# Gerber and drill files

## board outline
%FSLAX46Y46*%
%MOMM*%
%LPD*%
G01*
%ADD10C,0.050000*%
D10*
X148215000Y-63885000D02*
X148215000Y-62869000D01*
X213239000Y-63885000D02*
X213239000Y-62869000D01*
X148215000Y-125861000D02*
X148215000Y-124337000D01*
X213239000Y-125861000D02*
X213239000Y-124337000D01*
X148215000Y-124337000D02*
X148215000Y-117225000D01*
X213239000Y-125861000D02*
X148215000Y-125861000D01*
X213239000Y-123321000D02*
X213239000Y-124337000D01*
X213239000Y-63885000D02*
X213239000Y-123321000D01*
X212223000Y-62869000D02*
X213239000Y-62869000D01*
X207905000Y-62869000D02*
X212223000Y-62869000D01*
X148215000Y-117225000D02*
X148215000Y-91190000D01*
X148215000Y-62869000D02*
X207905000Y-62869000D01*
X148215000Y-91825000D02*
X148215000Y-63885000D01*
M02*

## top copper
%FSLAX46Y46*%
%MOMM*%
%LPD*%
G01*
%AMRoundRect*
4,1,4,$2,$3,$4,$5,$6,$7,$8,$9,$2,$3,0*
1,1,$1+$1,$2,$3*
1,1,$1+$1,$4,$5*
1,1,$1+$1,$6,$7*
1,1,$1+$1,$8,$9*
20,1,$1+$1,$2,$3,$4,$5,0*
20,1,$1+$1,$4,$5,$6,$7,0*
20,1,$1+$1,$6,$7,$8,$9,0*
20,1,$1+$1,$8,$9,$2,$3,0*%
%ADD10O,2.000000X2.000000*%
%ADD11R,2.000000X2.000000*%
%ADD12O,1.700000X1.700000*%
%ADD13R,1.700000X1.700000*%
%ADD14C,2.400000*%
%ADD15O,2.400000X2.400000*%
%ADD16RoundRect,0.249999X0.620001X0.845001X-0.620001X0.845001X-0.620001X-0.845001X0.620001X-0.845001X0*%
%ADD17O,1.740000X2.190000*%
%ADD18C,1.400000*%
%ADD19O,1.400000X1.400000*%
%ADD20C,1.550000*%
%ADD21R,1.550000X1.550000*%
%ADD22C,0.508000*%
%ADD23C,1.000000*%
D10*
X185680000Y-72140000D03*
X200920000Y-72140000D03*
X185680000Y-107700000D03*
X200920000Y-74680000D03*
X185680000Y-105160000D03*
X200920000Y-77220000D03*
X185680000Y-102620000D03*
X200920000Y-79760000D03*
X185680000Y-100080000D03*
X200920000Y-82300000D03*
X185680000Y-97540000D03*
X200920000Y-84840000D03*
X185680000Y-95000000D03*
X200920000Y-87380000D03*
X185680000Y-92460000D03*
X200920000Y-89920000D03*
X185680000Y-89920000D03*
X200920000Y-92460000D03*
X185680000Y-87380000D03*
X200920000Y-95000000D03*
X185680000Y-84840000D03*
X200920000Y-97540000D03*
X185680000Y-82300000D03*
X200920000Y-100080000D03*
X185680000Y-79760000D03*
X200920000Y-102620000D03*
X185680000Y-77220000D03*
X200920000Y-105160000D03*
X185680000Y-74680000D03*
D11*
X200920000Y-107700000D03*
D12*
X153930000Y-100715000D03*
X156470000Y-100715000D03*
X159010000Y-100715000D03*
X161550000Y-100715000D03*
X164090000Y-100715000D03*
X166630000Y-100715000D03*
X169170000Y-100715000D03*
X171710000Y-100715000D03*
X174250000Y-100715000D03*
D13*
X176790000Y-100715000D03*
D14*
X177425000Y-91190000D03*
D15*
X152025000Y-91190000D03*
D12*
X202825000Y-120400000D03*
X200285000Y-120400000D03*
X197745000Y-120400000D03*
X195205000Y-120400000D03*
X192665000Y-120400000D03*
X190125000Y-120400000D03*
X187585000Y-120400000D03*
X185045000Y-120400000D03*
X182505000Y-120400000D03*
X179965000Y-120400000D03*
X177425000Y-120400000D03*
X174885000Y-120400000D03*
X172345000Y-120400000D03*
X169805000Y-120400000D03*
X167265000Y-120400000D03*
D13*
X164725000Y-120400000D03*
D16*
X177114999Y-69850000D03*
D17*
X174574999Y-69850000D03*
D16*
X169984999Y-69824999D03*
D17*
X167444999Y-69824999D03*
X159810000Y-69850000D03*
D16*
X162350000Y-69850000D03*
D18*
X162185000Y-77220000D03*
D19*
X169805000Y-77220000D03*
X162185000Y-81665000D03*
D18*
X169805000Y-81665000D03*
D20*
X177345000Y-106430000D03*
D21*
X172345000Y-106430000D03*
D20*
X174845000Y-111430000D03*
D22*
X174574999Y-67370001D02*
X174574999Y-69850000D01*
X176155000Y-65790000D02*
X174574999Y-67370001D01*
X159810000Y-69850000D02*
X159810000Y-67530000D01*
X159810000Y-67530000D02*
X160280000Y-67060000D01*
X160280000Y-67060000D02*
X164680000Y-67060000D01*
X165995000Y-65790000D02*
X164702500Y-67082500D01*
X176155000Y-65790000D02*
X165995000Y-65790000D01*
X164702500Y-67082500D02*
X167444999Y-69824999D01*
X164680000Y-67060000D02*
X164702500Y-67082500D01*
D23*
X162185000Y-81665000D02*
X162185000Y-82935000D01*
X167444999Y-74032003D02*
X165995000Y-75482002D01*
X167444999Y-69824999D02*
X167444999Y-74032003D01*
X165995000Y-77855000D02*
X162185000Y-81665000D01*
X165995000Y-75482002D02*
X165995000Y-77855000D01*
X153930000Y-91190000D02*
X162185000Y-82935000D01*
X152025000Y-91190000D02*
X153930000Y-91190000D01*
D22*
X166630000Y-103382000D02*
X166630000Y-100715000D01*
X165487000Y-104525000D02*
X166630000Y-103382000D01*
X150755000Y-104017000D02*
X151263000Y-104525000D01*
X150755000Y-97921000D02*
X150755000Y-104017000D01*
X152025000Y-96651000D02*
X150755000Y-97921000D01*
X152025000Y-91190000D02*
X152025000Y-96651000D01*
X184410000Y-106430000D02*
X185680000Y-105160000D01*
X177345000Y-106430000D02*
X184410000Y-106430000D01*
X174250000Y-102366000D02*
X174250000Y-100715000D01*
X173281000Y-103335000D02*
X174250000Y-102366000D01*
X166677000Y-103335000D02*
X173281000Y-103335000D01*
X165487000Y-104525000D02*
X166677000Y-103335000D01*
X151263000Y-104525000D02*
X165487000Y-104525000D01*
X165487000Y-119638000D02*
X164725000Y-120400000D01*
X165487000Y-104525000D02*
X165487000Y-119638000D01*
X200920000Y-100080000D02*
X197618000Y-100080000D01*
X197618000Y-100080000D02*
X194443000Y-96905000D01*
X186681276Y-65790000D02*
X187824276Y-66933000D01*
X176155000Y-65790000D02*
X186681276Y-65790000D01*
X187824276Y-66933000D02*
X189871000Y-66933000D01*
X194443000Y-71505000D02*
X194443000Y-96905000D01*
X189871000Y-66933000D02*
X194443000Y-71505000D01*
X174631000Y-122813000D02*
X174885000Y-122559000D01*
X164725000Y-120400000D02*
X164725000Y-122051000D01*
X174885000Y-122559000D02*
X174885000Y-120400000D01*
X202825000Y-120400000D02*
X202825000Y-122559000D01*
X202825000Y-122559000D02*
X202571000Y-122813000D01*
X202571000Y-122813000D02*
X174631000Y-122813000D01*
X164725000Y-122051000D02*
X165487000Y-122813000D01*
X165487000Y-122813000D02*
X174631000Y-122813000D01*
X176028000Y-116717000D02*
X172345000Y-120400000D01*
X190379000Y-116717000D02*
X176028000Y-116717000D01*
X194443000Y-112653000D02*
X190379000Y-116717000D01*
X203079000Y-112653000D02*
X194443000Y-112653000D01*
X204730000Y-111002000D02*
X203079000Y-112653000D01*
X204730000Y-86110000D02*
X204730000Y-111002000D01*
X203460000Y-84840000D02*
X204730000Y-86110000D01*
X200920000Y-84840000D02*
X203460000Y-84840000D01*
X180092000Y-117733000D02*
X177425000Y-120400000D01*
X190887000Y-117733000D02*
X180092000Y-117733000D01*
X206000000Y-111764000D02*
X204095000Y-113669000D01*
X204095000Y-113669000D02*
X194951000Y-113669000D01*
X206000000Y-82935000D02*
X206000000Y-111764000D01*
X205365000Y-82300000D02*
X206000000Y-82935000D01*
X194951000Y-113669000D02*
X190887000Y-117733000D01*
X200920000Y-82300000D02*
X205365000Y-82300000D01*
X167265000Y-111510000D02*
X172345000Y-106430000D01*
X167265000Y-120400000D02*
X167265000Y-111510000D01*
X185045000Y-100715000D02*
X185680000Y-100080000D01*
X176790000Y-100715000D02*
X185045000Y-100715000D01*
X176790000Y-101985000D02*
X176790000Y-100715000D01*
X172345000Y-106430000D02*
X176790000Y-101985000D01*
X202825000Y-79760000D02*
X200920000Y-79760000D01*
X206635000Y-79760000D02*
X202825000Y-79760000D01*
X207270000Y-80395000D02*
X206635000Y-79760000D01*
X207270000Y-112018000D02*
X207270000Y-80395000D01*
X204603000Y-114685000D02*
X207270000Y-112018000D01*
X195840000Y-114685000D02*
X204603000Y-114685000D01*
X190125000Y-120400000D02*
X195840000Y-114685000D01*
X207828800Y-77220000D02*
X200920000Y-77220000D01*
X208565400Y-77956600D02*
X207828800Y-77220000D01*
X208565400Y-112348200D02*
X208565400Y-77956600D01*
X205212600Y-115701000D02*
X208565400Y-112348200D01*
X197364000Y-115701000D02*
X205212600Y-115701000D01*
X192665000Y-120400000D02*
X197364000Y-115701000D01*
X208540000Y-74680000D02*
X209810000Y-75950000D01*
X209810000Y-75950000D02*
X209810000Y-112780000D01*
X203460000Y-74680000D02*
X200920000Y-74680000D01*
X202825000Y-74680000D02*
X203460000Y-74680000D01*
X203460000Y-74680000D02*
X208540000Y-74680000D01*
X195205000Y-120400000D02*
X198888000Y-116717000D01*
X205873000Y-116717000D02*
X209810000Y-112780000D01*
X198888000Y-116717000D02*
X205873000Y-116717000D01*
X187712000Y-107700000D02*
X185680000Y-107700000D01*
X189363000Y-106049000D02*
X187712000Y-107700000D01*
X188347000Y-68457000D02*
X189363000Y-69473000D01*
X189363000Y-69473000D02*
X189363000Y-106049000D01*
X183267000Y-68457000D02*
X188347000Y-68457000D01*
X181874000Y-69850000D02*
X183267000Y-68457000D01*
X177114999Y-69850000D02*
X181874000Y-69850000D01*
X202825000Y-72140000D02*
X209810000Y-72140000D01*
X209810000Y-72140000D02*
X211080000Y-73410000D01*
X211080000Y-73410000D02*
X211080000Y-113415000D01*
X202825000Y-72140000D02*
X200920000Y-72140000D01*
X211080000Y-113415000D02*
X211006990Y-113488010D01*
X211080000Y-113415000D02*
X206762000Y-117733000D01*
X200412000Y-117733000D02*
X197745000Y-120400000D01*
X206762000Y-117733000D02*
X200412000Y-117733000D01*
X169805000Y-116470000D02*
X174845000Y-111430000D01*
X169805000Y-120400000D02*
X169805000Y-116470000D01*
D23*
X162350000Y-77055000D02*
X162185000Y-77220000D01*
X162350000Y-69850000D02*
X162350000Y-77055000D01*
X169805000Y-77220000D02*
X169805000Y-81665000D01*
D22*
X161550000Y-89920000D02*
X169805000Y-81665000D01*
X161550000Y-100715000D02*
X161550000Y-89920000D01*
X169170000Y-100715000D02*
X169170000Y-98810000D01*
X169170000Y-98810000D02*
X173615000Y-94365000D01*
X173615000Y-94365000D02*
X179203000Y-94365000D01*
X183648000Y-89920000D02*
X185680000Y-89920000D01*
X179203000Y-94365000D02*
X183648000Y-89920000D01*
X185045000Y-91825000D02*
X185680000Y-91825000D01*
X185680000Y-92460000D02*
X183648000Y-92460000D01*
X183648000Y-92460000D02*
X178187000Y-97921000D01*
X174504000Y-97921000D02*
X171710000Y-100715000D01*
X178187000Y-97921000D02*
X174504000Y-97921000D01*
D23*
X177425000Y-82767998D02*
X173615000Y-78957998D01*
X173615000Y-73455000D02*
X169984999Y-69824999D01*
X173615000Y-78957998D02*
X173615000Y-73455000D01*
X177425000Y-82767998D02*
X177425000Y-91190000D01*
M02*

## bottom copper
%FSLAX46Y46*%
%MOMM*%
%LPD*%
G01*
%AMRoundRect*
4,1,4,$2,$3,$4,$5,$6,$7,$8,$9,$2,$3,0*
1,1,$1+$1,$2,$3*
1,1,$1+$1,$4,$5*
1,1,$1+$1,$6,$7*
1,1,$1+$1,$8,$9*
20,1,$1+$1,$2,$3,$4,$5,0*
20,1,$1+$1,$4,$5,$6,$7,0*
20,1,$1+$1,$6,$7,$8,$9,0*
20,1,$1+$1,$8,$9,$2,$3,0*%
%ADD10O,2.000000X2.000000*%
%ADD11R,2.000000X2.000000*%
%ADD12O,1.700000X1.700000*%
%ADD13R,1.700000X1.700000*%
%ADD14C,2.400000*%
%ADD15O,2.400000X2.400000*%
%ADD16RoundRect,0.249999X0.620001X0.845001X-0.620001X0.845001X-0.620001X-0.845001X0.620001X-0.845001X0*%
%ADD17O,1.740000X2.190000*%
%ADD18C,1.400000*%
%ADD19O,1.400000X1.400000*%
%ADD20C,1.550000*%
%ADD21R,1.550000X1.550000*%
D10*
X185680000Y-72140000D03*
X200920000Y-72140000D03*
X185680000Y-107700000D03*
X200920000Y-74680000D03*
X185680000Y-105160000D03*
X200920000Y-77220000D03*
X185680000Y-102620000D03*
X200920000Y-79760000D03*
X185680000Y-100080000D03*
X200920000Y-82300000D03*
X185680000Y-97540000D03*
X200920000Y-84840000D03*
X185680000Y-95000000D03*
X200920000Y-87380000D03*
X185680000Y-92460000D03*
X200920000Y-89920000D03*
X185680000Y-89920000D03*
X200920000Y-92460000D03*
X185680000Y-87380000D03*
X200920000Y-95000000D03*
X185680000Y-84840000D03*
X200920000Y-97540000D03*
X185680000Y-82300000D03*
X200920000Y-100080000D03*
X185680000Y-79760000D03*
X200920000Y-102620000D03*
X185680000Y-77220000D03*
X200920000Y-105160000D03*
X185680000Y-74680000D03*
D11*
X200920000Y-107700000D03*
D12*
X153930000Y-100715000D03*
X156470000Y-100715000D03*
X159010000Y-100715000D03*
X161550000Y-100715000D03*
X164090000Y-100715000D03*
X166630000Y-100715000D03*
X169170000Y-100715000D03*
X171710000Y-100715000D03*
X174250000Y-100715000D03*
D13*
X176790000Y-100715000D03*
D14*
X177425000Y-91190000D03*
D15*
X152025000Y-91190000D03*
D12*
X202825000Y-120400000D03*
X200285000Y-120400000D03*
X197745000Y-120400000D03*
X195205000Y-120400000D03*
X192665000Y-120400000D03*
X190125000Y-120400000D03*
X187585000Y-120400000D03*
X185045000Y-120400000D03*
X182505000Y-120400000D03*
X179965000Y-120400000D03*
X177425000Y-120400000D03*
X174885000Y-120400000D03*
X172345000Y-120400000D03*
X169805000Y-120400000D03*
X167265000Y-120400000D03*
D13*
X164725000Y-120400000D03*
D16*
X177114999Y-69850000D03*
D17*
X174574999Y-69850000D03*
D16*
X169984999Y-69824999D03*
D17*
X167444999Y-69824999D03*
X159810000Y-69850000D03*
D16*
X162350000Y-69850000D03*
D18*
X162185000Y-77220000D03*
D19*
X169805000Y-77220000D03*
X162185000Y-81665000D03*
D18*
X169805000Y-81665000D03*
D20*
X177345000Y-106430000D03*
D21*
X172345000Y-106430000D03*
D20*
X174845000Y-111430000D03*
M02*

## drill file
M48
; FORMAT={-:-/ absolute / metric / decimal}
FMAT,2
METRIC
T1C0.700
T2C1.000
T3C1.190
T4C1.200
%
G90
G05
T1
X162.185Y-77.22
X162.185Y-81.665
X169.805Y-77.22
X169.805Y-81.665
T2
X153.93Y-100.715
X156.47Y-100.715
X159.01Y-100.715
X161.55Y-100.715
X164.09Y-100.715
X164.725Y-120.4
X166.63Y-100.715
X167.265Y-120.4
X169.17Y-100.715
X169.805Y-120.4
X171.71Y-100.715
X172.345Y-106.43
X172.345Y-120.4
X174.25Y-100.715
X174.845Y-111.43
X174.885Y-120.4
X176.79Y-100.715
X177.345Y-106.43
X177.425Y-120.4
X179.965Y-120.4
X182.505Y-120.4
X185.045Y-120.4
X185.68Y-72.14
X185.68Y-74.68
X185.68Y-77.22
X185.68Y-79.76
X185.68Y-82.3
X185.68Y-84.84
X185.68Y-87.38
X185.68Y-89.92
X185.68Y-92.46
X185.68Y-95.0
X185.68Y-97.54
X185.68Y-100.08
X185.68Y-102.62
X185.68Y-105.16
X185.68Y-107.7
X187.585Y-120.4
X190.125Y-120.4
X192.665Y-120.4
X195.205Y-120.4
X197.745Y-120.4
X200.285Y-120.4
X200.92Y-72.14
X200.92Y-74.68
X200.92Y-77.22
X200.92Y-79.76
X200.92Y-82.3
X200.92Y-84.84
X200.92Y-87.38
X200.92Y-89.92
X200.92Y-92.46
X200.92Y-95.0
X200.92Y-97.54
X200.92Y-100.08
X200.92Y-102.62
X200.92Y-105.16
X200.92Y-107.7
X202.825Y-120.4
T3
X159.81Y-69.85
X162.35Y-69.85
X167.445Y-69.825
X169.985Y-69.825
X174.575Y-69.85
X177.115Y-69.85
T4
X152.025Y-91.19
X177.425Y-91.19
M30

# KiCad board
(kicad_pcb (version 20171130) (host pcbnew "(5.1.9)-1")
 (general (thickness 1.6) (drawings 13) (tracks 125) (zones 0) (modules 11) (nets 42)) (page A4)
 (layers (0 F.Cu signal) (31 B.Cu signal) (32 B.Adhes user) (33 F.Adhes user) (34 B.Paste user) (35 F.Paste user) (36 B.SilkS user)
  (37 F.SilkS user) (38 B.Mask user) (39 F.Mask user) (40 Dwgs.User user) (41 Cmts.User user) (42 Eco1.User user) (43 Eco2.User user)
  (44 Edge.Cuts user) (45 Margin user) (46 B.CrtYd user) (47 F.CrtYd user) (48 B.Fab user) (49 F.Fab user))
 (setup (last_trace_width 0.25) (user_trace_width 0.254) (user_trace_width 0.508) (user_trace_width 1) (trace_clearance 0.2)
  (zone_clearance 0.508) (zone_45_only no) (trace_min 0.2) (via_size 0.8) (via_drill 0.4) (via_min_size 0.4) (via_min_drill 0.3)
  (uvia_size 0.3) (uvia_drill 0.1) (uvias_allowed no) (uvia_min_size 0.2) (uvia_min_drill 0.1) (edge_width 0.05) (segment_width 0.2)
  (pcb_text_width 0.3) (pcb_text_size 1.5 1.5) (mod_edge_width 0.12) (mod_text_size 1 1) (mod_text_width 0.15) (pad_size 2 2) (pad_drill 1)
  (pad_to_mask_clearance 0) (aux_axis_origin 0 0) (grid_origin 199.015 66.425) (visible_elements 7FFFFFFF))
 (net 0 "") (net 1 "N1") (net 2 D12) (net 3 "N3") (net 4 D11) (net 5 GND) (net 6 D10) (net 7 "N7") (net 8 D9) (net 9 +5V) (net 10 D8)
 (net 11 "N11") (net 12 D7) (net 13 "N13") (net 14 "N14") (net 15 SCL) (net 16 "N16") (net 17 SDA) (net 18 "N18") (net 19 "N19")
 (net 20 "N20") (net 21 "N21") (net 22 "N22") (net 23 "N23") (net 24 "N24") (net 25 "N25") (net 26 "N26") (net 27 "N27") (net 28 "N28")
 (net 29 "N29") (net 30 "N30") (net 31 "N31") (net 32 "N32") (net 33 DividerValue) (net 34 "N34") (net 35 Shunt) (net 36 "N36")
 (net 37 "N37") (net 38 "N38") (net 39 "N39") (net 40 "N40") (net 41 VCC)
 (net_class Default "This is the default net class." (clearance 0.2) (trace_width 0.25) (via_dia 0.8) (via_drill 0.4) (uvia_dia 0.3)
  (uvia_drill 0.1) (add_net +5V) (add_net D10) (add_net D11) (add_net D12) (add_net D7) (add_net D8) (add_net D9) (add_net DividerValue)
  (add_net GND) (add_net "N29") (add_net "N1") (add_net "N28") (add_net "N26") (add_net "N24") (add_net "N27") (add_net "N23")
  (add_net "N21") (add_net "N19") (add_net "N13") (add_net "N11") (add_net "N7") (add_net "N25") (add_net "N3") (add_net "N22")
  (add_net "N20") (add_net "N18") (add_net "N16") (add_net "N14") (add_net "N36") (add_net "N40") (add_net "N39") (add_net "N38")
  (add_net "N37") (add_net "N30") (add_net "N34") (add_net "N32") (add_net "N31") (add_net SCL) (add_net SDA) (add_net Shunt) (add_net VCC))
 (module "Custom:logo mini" (layer F.Cu) (at 157.359 114.685)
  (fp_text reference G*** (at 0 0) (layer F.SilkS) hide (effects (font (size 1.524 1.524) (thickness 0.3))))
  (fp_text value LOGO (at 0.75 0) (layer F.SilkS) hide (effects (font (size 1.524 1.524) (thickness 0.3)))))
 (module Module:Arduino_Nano (layer F.Cu) (at 200.92 107.7 180)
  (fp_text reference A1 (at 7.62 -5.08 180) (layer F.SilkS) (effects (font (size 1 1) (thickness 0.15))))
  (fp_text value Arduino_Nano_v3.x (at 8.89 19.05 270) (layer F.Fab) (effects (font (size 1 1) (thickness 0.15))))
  (pad 16 thru_hole oval (at 15.24 35.56 180) (size 2 2) (drill 1) (layers *.Cu *.Mask) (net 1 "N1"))
  (pad 15 thru_hole oval (at 0 35.56 180) (size 2 2) (drill 1) (layers *.Cu *.Mask) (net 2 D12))
  (pad 30 thru_hole oval (at 15.24 0 180) (size 2 2) (drill 1) (layers *.Cu *.Mask) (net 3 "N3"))
  (pad 14 thru_hole oval (at 0 33.02 180) (size 2 2) (drill 1) (layers *.Cu *.Mask) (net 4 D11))
  (pad 29 thru_hole oval (at 15.24 2.54 180) (size 2 2) (drill 1) (layers *.Cu *.Mask) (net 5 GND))
  (pad 13 thru_hole oval (at 0 30.48 180) (size 2 2) (drill 1) (layers *.Cu *.Mask) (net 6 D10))
  (pad 28 thru_hole oval (at 15.24 5.08 180) (size 2 2) (drill 1) (layers *.Cu *.Mask) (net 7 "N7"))
  (pad 12 thru_hole oval (at 0 27.94 180) (size 2 2) (drill 1) (layers *.Cu *.Mask) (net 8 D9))
  (pad 27 thru_hole oval (at 15.24 7.62 180) (size 2 2) (drill 1) (layers *.Cu *.Mask) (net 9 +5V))
  (pad 11 thru_hole oval (at 0 25.4 180) (size 2 2) (drill 1) (layers *.Cu *.Mask) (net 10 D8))
  (pad 26 thru_hole oval (at 15.24 10.16 180) (size 2 2) (drill 1) (layers *.Cu *.Mask) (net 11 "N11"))
  (pad 10 thru_hole oval (at 0 22.86 180) (size 2 2) (drill 1) (layers *.Cu *.Mask) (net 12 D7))
  (pad 25 thru_hole oval (at 15.24 12.7 180) (size 2 2) (drill 1) (layers *.Cu *.Mask) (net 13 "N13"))
  (pad 9 thru_hole oval (at 0 20.32 180) (size 2 2) (drill 1) (layers *.Cu *.Mask) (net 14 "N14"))
  (pad 24 thru_hole oval (at 15.24 15.24 180) (size 2 2) (drill 1) (layers *.Cu *.Mask) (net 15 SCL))
  (pad 8 thru_hole oval (at 0 17.78 180) (size 2 2) (drill 1) (layers *.Cu *.Mask) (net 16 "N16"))
  (pad 23 thru_hole oval (at 15.24 17.78 180) (size 2 2) (drill 1) (layers *.Cu *.Mask) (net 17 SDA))
  (pad 7 thru_hole oval (at 0 15.24 180) (size 2 2) (drill 1) (layers *.Cu *.Mask) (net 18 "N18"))
  (pad 22 thru_hole oval (at 15.24 20.32 180) (size 2 2) (drill 1) (layers *.Cu *.Mask) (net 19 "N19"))
  (pad 6 thru_hole oval (at 0 12.7 180) (size 2 2) (drill 1) (layers *.Cu *.Mask) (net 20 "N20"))
  (pad 21 thru_hole oval (at 15.24 22.86 180) (size 2 2) (drill 1) (layers *.Cu *.Mask) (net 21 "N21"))
  (pad 5 thru_hole oval (at 0 10.16 180) (size 2 2) (drill 1) (layers *.Cu *.Mask) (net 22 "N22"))
  (pad 20 thru_hole oval (at 15.24 25.4 180) (size 2 2) (drill 1) (layers *.Cu *.Mask) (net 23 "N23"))
  (pad 4 thru_hole oval (at 0 7.62 180) (size 2 2) (drill 1) (layers *.Cu *.Mask) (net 5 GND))
  (pad 19 thru_hole oval (at 15.24 27.94 180) (size 2 2) (drill 1) (layers *.Cu *.Mask) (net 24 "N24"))
  (pad 3 thru_hole oval (at 0 5.08 180) (size 2 2) (drill 1) (layers *.Cu *.Mask) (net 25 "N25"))
  (pad 18 thru_hole oval (at 15.24 30.48 180) (size 2 2) (drill 1) (layers *.Cu *.Mask) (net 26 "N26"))
  (pad 2 thru_hole oval (at 0 2.54 180) (size 2 2) (drill 1) (layers *.Cu *.Mask) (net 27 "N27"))
  (pad 17 thru_hole oval (at 15.24 33.02 180) (size 2 2) (drill 1) (layers *.Cu *.Mask) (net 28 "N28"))
  (pad 1 thru_hole rect (at 0 0 180) (size 2 2) (drill 1) (layers *.Cu *.Mask) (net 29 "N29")))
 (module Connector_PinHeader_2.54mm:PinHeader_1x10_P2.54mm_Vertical (layer F.Cu) (at 176.79 100.715 270)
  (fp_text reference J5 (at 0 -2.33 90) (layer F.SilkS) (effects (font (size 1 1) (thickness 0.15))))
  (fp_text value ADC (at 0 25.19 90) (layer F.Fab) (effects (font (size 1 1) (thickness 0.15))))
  (pad 10 thru_hole oval (at 0 22.86 270) (size 1.7 1.7) (drill 1) (layers *.Cu *.Mask) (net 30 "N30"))
  (pad 9 thru_hole oval (at 0 20.32 270) (size 1.7 1.7) (drill 1) (layers *.Cu *.Mask) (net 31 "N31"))
  (pad 8 thru_hole oval (at 0 17.78 270) (size 1.7 1.7) (drill 1) (layers *.Cu *.Mask) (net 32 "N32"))
  (pad 7 thru_hole oval (at 0 15.24 270) (size 1.7 1.7) (drill 1) (layers *.Cu *.Mask) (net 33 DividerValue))
  (pad 6 thru_hole oval (at 0 12.7 270) (size 1.7 1.7) (drill 1) (layers *.Cu *.Mask) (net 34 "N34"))
  (pad 5 thru_hole oval (at 0 10.16 270) (size 1.7 1.7) (drill 1) (layers *.Cu *.Mask) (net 5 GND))
  (pad 4 thru_hole oval (at 0 7.62 270) (size 1.7 1.7) (drill 1) (layers *.Cu *.Mask) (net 17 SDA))
  (pad 3 thru_hole oval (at 0 5.08 270) (size 1.7 1.7) (drill 1) (layers *.Cu *.Mask) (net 15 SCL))
  (pad 2 thru_hole oval (at 0 2.54 270) (size 1.7 1.7) (drill 1) (layers *.Cu *.Mask) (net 5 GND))
  (pad 1 thru_hole rect (at 0 0 270) (size 1.7 1.7) (drill 1) (layers *.Cu *.Mask) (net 9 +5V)))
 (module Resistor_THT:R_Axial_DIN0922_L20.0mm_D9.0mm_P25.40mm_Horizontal (layer F.Cu) (at 177.425 91.19 180)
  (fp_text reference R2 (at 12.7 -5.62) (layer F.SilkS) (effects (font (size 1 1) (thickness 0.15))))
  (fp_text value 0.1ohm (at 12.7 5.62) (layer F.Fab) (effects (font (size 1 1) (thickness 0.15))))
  (pad 1 thru_hole circle (at 0 0 180) (size 2.4 2.4) (drill 1.2) (layers *.Cu *.Mask) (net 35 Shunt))
  (pad 2 thru_hole oval (at 25.4 0 180) (size 2.4 2.4) (drill 1.2) (layers *.Cu *.Mask) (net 5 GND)))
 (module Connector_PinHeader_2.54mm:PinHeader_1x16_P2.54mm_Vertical (layer F.Cu) (at 164.725 120.4 90)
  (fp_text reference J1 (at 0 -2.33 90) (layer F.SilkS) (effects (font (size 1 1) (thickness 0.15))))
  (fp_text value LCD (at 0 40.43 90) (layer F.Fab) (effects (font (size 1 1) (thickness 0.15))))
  (pad 16 thru_hole oval (at 0 38.1 90) (size 1.7 1.7) (drill 1) (layers *.Cu *.Mask) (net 5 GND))
  (pad 15 thru_hole oval (at 0 35.56 90) (size 1.7 1.7) (drill 1) (layers *.Cu *.Mask) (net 9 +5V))
  (pad 14 thru_hole oval (at 0 33.02 90) (size 1.7 1.7) (drill 1) (layers *.Cu *.Mask) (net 2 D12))
  (pad 13 thru_hole oval (at 0 30.48 90) (size 1.7 1.7) (drill 1) (layers *.Cu *.Mask) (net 4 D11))
  (pad 12 thru_hole oval (at 0 27.94 90) (size 1.7 1.7) (drill 1) (layers *.Cu *.Mask) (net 6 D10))
  (pad 11 thru_hole oval (at 0 25.4 90) (size 1.7 1.7) (drill 1) (layers *.Cu *.Mask) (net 8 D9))
  (pad 10 thru_hole oval (at 0 22.86 90) (size 1.7 1.7) (drill 1) (layers *.Cu *.Mask) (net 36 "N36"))
  (pad 9 thru_hole oval (at 0 20.32 90) (size 1.7 1.7) (drill 1) (layers *.Cu *.Mask) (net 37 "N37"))
  (pad 8 thru_hole oval (at 0 17.78 90) (size 1.7 1.7) (drill 1) (layers *.Cu *.Mask) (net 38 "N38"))
  (pad 7 thru_hole oval (at 0 15.24 90) (size 1.7 1.7) (drill 1) (layers *.Cu *.Mask) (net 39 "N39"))
  (pad 6 thru_hole oval (at 0 12.7 90) (size 1.7 1.7) (drill 1) (layers *.Cu *.Mask) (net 10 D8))
  (pad 5 thru_hole oval (at 0 10.16 90) (size 1.7 1.7) (drill 1) (layers *.Cu *.Mask) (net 5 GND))
  (pad 4 thru_hole oval (at 0 7.62 90) (size 1.7 1.7) (drill 1) (layers *.Cu *.Mask) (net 12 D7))
  (pad 3 thru_hole oval (at 0 5.08 90) (size 1.7 1.7) (drill 1) (layers *.Cu *.Mask) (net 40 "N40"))
  (pad 2 thru_hole oval (at 0 2.54 90) (size 1.7 1.7) (drill 1) (layers *.Cu *.Mask) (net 9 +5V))
  (pad 1 thru_hole rect (at 0 0 90) (size 1.7 1.7) (drill 1) (layers *.Cu *.Mask) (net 5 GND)))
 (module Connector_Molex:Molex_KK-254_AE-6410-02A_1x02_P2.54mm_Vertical (layer F.Cu) (at 177.114999 69.85 180)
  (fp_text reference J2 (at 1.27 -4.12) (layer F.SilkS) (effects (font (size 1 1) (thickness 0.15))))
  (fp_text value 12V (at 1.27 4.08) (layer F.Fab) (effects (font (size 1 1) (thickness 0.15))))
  (pad 1 thru_hole roundrect (at 0 0 180) (size 1.74 2.19) (drill 1.19) (layers *.Cu *.Mask) (roundrect_rratio 0.1436775862068966)
   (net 3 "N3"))
  (pad 2 thru_hole oval (at 2.54 0 180) (size 1.74 2.19) (drill 1.19) (layers *.Cu *.Mask) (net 5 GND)))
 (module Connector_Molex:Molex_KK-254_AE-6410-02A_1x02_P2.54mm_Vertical (layer F.Cu) (at 169.984999 69.824999 180)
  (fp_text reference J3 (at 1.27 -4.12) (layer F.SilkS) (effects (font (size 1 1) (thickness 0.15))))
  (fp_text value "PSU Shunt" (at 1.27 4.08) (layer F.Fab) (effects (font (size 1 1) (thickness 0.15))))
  (pad 1 thru_hole roundrect (at 0 0 180) (size 1.74 2.19) (drill 1.19) (layers *.Cu *.Mask) (roundrect_rratio 0.1436775862068966)
   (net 35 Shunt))
  (pad 2 thru_hole oval (at 2.54 0 180) (size 1.74 2.19) (drill 1.19) (layers *.Cu *.Mask) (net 5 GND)))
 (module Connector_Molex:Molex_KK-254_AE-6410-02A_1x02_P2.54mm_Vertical (layer F.Cu) (at 162.35 69.85 180)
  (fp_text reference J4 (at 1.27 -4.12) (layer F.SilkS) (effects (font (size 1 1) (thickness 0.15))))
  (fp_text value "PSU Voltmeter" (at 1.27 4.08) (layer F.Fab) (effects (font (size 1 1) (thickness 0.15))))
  (pad 2 thru_hole oval (at 2.54 0 180) (size 1.74 2.19) (drill 1.19) (layers *.Cu *.Mask) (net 5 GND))
  (pad 1 thru_hole roundrect (at 0 0 180) (size 1.74 2.19) (drill 1.19) (layers *.Cu *.Mask) (roundrect_rratio 0.1436775862068966)
   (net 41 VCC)))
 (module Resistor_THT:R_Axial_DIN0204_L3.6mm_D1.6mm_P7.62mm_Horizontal (layer F.Cu) (at 162.185 77.22)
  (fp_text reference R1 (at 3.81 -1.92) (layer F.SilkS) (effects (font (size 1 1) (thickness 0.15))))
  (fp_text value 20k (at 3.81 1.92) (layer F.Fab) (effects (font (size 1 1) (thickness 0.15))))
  (pad 1 thru_hole circle (at 0 0) (size 1.4 1.4) (drill 0.7) (layers *.Cu *.Mask) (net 41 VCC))
  (pad 2 thru_hole oval (at 7.62 0) (size 1.4 1.4) (drill 0.7) (layers *.Cu *.Mask) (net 33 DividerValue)))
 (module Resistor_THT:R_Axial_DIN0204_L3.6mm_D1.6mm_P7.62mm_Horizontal (layer F.Cu) (at 169.805 81.665 180)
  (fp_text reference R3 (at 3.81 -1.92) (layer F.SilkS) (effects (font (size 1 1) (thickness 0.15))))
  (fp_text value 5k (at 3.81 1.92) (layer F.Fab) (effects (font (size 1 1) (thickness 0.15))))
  (pad 2 thru_hole oval (at 7.62 0 180) (size 1.4 1.4) (drill 0.7) (layers *.Cu *.Mask) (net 5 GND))
  (pad 1 thru_hole circle (at 0 0 180) (size 1.4 1.4) (drill 0.7) (layers *.Cu *.Mask) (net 33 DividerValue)))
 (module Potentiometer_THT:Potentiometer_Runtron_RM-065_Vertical (layer F.Cu) (at 172.345 106.43)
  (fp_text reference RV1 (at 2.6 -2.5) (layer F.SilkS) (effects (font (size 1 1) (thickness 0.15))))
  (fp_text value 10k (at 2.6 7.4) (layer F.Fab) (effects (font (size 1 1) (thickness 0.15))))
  (pad 3 thru_hole circle (at 5 0) (size 1.55 1.55) (drill 1) (layers *.Cu *.Mask) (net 5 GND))
  (pad 1 thru_hole rect (at 0 0) (size 1.55 1.55) (drill 1) (layers *.Cu *.Mask) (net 9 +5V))
  (pad 2 thru_hole circle (at 2.5 5) (size 1.55 1.55) (drill 1) (layers *.Cu *.Mask) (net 40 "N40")))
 (gr_line (start 148.215 63.885) (end 148.215 62.869) (layer Edge.Cuts) (width 0.05))
 (gr_line (start 213.239 63.885) (end 213.239 62.869) (layer Edge.Cuts) (width 0.05))
 (gr_line (start 148.215 125.861) (end 148.215 124.337) (layer Edge.Cuts) (width 0.05))
 (gr_line (start 213.239 125.861) (end 213.239 124.337) (layer Edge.Cuts) (width 0.05))
 (gr_line (start 148.215 124.337) (end 148.215 117.225) (layer Edge.Cuts) (width 0.05))
 (gr_line (start 213.239 125.861) (end 148.215 125.861) (layer Edge.Cuts) (width 0.05))
 (gr_line (start 213.239 123.321) (end 213.239 124.337) (layer Edge.Cuts) (width 0.05))
 (gr_line (start 213.239 63.885) (end 213.239 123.321) (layer Edge.Cuts) (width 0.05))
 (gr_line (start 212.223 62.869) (end 213.239 62.869) (layer Edge.Cuts) (width 0.05))
 (gr_line (start 207.905 62.869) (end 212.223 62.869) (layer Edge.Cuts) (width 0.05))
 (gr_line (start 148.215 117.225) (end 148.215 91.19) (layer Edge.Cuts) (width 0.05))
 (gr_line (start 148.215 62.869) (end 207.905 62.869) (layer Edge.Cuts) (width 0.05))
 (gr_line (start 148.215 91.825) (end 148.215 63.885) (layer Edge.Cuts) (width 0.05))
 (segment (start 174.574999 67.370001) (end 174.574999 69.85) (width 0.508) (layer F.Cu) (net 5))
 (segment (start 176.155 65.79) (end 174.574999 67.370001) (width 0.508) (layer F.Cu) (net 5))
 (segment (start 159.81 69.85) (end 159.81 67.53) (width 0.508) (layer F.Cu) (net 5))
 (segment (start 159.81 67.53) (end 160.28 67.06) (width 0.508) (layer F.Cu) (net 5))
 (segment (start 160.28 67.06) (end 164.68 67.06) (width 0.508) (layer F.Cu) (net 5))
 (segment (start 165.995 65.79) (end 164.7025 67.0825) (width 0.508) (layer F.Cu) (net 5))
 (segment (start 176.155 65.79) (end 165.995 65.79) (width 0.508) (layer F.Cu) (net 5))
 (segment (start 164.7025 67.0825) (end 167.444999 69.824999) (width 0.508) (layer F.Cu) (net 5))
 (segment (start 164.68 67.06) (end 164.7025 67.0825) (width 0.508) (layer F.Cu) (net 5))
 (segment (start 162.185 81.665) (end 162.185 82.935) (width 1) (layer F.Cu) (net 5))
 (segment (start 167.444999 74.032003) (end 165.995 75.482002) (width 1) (layer F.Cu) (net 5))
 (segment (start 167.444999 69.824999) (end 167.444999 74.032003) (width 1) (layer F.Cu) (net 5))
 (segment (start 165.995 77.855) (end 162.185 81.665) (width 1) (layer F.Cu) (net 5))
 (segment (start 165.995 75.482002) (end 165.995 77.855) (width 1) (layer F.Cu) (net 5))
 (segment (start 153.93 91.19) (end 162.185 82.935) (width 1) (layer F.Cu) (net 5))
 (segment (start 152.025 91.19) (end 153.93 91.19) (width 1) (layer F.Cu) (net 5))
 (segment (start 166.63 103.382) (end 166.63 100.715) (width 0.508) (layer F.Cu) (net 5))
 (segment (start 165.487 104.525) (end 166.63 103.382) (width 0.508) (layer F.Cu) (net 5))
 (segment (start 150.755 104.017) (end 151.263 104.525) (width 0.508) (layer F.Cu) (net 5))
 (segment (start 150.755 97.921) (end 150.755 104.017) (width 0.508) (layer F.Cu) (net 5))
 (segment (start 152.025 96.651) (end 150.755 97.921) (width 0.508) (layer F.Cu) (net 5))
 (segment (start 152.025 91.19) (end 152.025 96.651) (width 0.508) (layer F.Cu) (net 5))
 (segment (start 184.41 106.43) (end 185.68 105.16) (width 0.508) (layer F.Cu) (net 5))
 (segment (start 177.345 106.43) (end 184.41 106.43) (width 0.508) (layer F.Cu) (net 5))
 (segment (start 174.25 102.366) (end 174.25 100.715) (width 0.508) (layer F.Cu) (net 5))
 (segment (start 173.281 103.335) (end 174.25 102.366) (width 0.508) (layer F.Cu) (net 5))
 (segment (start 166.677 103.335) (end 173.281 103.335) (width 0.508) (layer F.Cu) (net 5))
 (segment (start 165.487 104.525) (end 166.677 103.335) (width 0.508) (layer F.Cu) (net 5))
 (segment (start 151.263 104.525) (end 165.487 104.525) (width 0.508) (layer F.Cu) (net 5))
 (segment (start 165.487 119.638) (end 164.725 120.4) (width 0.508) (layer F.Cu) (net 5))
 (segment (start 165.487 104.525) (end 165.487 119.638) (width 0.508) (layer F.Cu) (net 5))
 (segment (start 200.92 100.08) (end 197.618 100.08) (width 0.508) (layer F.Cu) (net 5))
 (segment (start 197.618 100.08) (end 194.443 96.905) (width 0.508) (layer F.Cu) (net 5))
 (segment (start 186.681276 65.79) (end 187.824276 66.933) (width 0.508) (layer F.Cu) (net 5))
 (segment (start 176.155 65.79) (end 186.681276 65.79) (width 0.508) (layer F.Cu) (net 5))
 (segment (start 187.824276 66.933) (end 189.871 66.933) (width 0.508) (layer F.Cu) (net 5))
 (segment (start 194.443 71.505) (end 194.443 96.905) (width 0.508) (layer F.Cu) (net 5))
 (segment (start 189.871 66.933) (end 194.443 71.505) (width 0.508) (layer F.Cu) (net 5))
 (segment (start 174.631 122.813) (end 174.885 122.559) (width 0.508) (layer F.Cu) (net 5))
 (segment (start 164.725 120.4) (end 164.725 122.051) (width 0.508) (layer F.Cu) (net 5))
 (segment (start 174.885 122.559) (end 174.885 120.4) (width 0.508) (layer F.Cu) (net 5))
 (segment (start 202.825 120.4) (end 202.825 122.559) (width 0.508) (layer F.Cu) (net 5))
 (segment (start 202.825 122.559) (end 202.571 122.813) (width 0.508) (layer F.Cu) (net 5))
 (segment (start 202.571 122.813) (end 174.631 122.813) (width 0.508) (layer F.Cu) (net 5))
 (segment (start 164.725 122.051) (end 165.487 122.813) (width 0.508) (layer F.Cu) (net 5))
 (segment (start 165.487 122.813) (end 174.631 122.813) (width 0.508) (layer F.Cu) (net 5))
 (segment (start 176.028 116.717) (end 172.345 120.4) (width 0.508) (layer F.Cu) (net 12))
 (segment (start 190.379 116.717) (end 176.028 116.717) (width 0.508) (layer F.Cu) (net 12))
 (segment (start 194.443 112.653) (end 190.379 116.717) (width 0.508) (layer F.Cu) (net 12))
 (segment (start 203.079 112.653) (end 194.443 112.653) (width 0.508) (layer F.Cu) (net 12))
 (segment (start 204.73 111.002) (end 203.079 112.653) (width 0.508) (layer F.Cu) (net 12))
 (segment (start 204.73 86.11) (end 204.73 111.002) (width 0.508) (layer F.Cu) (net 12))
 (segment (start 203.46 84.84) (end 204.73 86.11) (width 0.508) (layer F.Cu) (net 12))
 (segment (start 200.92 84.84) (end 203.46 84.84) (width 0.508) (layer F.Cu) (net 12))
 (segment (start 180.092 117.733) (end 177.425 120.4) (width 0.508) (layer F.Cu) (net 10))
 (segment (start 190.887 117.733) (end 180.092 117.733) (width 0.508) (layer F.Cu) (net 10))
 (segment (start 206 111.764) (end 204.095 113.669) (width 0.508) (layer F.Cu) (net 10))
 (segment (start 204.095 113.669) (end 194.951 113.669) (width 0.508) (layer F.Cu) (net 10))
 (segment (start 206 82.935) (end 206 111.764) (width 0.508) (layer F.Cu) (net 10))
 (segment (start 205.365 82.3) (end 206 82.935) (width 0.508) (layer F.Cu) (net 10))
 (segment (start 194.951 113.669) (end 190.887 117.733) (width 0.508) (layer F.Cu) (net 10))
 (segment (start 200.92 82.3) (end 205.365 82.3) (width 0.508) (layer F.Cu) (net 10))
 (segment (start 167.265 111.51) (end 172.345 106.43) (width 0.508) (layer F.Cu) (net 9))
 (segment (start 167.265 120.4) (end 167.265 111.51) (width 0.508) (layer F.Cu) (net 9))
 (segment (start 185.045 100.715) (end 185.68 100.08) (width 0.508) (layer F.Cu) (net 9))
 (segment (start 176.79 100.715) (end 185.045 100.715) (width 0.508) (layer F.Cu) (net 9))
 (segment (start 176.79 101.985) (end 176.79 100.715) (width 0.508) (layer F.Cu) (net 9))
 (segment (start 172.345 106.43) (end 176.79 101.985) (width 0.508) (layer F.Cu) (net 9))
 (segment (start 202.825 79.76) (end 200.92 79.76) (width 0.508) (layer F.Cu) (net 8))
 (segment (start 206.635 79.76) (end 202.825 79.76) (width 0.508) (layer F.Cu) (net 8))
 (segment (start 207.27 80.395) (end 206.635 79.76) (width 0.508) (layer F.Cu) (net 8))
 (segment (start 207.27 112.018) (end 207.27 80.395) (width 0.508) (layer F.Cu) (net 8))
 (segment (start 204.603 114.685) (end 207.27 112.018) (width 0.508) (layer F.Cu) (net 8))
 (segment (start 195.84 114.685) (end 204.603 114.685) (width 0.508) (layer F.Cu) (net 8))
 (segment (start 190.125 120.4) (end 195.84 114.685) (width 0.508) (layer F.Cu) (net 8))
 (segment (start 207.8288 77.22) (end 200.92 77.22) (width 0.508) (layer F.Cu) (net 6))
 (segment (start 208.5654 77.9566) (end 207.8288 77.22) (width 0.508) (layer F.Cu) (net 6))
 (segment (start 208.5654 112.3482) (end 208.5654 77.9566) (width 0.508) (layer F.Cu) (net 6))
 (segment (start 205.2126 115.701) (end 208.5654 112.3482) (width 0.508) (layer F.Cu) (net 6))
 (segment (start 197.364 115.701) (end 205.2126 115.701) (width 0.508) (layer F.Cu) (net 6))
 (segment (start 192.665 120.4) (end 197.364 115.701) (width 0.508) (layer F.Cu) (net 6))
 (segment (start 208.54 74.68) (end 209.81 75.95) (width 0.508) (layer F.Cu) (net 4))
 (segment (start 209.81 75.95) (end 209.81 112.78) (width 0.508) (layer F.Cu) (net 4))
 (segment (start 203.46 74.68) (end 200.92 74.68) (width 0.508) (layer F.Cu) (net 4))
 (segment (start 202.825 74.68) (end 203.46 74.68) (width 0.508) (layer F.Cu) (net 4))
 (segment (start 203.46 74.68) (end 208.54 74.68) (width 0.508) (layer F.Cu) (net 4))
 (segment (start 195.205 120.4) (end 198.888 116.717) (width 0.508) (layer F.Cu) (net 4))
 (segment (start 205.873 116.717) (end 209.81 112.78) (width 0.508) (layer F.Cu) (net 4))
 (segment (start 198.888 116.717) (end 205.873 116.717) (width 0.508) (layer F.Cu) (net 4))
 (segment (start 187.712 107.7) (end 185.68 107.7) (width 0.508) (layer F.Cu) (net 3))
 (segment (start 189.363 106.049) (end 187.712 107.7) (width 0.508) (layer F.Cu) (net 3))
 (segment (start 188.347 68.457) (end 189.363 69.473) (width 0.508) (layer F.Cu) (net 3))
 (segment (start 189.363 69.473) (end 189.363 106.049) (width 0.508) (layer F.Cu) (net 3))
 (segment (start 183.267 68.457) (end 188.347 68.457) (width 0.508) (layer F.Cu) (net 3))
 (segment (start 181.874 69.85) (end 183.267 68.457) (width 0.508) (layer F.Cu) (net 3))
 (segment (start 177.114999 69.85) (end 181.874 69.85) (width 0.508) (layer F.Cu) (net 3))
 (segment (start 202.825 72.14) (end 209.81 72.14) (width 0.508) (layer F.Cu) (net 2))
 (segment (start 209.81 72.14) (end 211.08 73.41) (width 0.508) (layer F.Cu) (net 2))
 (segment (start 211.08 73.41) (end 211.08 113.415) (width 0.508) (layer F.Cu) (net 2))
 (segment (start 202.825 72.14) (end 200.92 72.14) (width 0.508) (layer F.Cu) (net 2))
 (segment (start 211.08 113.415) (end 211.00699 113.48801) (width 0.508) (layer F.Cu) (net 2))
 (segment (start 211.08 113.415) (end 206.762 117.733) (width 0.508) (layer F.Cu) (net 2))
 (segment (start 200.412 117.733) (end 197.745 120.4) (width 0.508) (layer F.Cu) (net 2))
 (segment (start 206.762 117.733) (end 200.412 117.733) (width 0.508) (layer F.Cu) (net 2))
 (segment (start 169.805 116.47) (end 174.845 111.43) (width 0.508) (layer F.Cu) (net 40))
 (segment (start 169.805 120.4) (end 169.805 116.47) (width 0.508) (layer F.Cu) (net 40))
 (segment (start 162.35 77.055) (end 162.185 77.22) (width 1) (layer F.Cu) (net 41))
 (segment (start 162.35 69.85) (end 162.35 77.055) (width 1) (layer F.Cu) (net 41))
 (segment (start 169.805 77.22) (end 169.805 81.665) (width 1) (layer F.Cu) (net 33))
 (segment (start 161.55 89.92) (end 169.805 81.665) (width 0.508) (layer F.Cu) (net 33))
 (segment (start 161.55 100.715) (end 161.55 89.92) (width 0.508) (layer F.Cu) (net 33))
 (segment (start 169.17 100.715) (end 169.17 98.81) (width 0.508) (layer F.Cu) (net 17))
 (segment (start 169.17 98.81) (end 173.615 94.365) (width 0.508) (layer F.Cu) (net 17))
 (segment (start 173.615 94.365) (end 179.203 94.365) (width 0.508) (layer F.Cu) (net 17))
 (segment (start 183.648 89.92) (end 185.68 89.92) (width 0.508) (layer F.Cu) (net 17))
 (segment (start 179.203 94.365) (end 183.648 89.92) (width 0.508) (layer F.Cu) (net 17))
 (segment (start 185.045 91.825) (end 185.68 91.825) (width 0.508) (layer F.Cu) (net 15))
 (segment (start 185.68 92.46) (end 183.648 92.46) (width 0.508) (layer F.Cu) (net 15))
 (segment (start 183.648 92.46) (end 178.187 97.921) (width 0.508) (layer F.Cu) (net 15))
 (segment (start 174.504 97.921) (end 171.71 100.715) (width 0.508) (layer F.Cu) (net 15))
 (segment (start 178.187 97.921) (end 174.504 97.921) (width 0.508) (layer F.Cu) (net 15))
 (segment (start 177.425 82.767998) (end 173.615 78.957998) (width 1) (layer F.Cu) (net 35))
 (segment (start 173.615 73.455) (end 169.984999 69.824999) (width 1) (layer F.Cu) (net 35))
 (segment (start 173.615 78.957998) (end 173.615 73.455) (width 1) (layer F.Cu) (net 35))
 (segment (start 177.425 82.767998) (end 177.425 91.19) (width 1) (layer F.Cu) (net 35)))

